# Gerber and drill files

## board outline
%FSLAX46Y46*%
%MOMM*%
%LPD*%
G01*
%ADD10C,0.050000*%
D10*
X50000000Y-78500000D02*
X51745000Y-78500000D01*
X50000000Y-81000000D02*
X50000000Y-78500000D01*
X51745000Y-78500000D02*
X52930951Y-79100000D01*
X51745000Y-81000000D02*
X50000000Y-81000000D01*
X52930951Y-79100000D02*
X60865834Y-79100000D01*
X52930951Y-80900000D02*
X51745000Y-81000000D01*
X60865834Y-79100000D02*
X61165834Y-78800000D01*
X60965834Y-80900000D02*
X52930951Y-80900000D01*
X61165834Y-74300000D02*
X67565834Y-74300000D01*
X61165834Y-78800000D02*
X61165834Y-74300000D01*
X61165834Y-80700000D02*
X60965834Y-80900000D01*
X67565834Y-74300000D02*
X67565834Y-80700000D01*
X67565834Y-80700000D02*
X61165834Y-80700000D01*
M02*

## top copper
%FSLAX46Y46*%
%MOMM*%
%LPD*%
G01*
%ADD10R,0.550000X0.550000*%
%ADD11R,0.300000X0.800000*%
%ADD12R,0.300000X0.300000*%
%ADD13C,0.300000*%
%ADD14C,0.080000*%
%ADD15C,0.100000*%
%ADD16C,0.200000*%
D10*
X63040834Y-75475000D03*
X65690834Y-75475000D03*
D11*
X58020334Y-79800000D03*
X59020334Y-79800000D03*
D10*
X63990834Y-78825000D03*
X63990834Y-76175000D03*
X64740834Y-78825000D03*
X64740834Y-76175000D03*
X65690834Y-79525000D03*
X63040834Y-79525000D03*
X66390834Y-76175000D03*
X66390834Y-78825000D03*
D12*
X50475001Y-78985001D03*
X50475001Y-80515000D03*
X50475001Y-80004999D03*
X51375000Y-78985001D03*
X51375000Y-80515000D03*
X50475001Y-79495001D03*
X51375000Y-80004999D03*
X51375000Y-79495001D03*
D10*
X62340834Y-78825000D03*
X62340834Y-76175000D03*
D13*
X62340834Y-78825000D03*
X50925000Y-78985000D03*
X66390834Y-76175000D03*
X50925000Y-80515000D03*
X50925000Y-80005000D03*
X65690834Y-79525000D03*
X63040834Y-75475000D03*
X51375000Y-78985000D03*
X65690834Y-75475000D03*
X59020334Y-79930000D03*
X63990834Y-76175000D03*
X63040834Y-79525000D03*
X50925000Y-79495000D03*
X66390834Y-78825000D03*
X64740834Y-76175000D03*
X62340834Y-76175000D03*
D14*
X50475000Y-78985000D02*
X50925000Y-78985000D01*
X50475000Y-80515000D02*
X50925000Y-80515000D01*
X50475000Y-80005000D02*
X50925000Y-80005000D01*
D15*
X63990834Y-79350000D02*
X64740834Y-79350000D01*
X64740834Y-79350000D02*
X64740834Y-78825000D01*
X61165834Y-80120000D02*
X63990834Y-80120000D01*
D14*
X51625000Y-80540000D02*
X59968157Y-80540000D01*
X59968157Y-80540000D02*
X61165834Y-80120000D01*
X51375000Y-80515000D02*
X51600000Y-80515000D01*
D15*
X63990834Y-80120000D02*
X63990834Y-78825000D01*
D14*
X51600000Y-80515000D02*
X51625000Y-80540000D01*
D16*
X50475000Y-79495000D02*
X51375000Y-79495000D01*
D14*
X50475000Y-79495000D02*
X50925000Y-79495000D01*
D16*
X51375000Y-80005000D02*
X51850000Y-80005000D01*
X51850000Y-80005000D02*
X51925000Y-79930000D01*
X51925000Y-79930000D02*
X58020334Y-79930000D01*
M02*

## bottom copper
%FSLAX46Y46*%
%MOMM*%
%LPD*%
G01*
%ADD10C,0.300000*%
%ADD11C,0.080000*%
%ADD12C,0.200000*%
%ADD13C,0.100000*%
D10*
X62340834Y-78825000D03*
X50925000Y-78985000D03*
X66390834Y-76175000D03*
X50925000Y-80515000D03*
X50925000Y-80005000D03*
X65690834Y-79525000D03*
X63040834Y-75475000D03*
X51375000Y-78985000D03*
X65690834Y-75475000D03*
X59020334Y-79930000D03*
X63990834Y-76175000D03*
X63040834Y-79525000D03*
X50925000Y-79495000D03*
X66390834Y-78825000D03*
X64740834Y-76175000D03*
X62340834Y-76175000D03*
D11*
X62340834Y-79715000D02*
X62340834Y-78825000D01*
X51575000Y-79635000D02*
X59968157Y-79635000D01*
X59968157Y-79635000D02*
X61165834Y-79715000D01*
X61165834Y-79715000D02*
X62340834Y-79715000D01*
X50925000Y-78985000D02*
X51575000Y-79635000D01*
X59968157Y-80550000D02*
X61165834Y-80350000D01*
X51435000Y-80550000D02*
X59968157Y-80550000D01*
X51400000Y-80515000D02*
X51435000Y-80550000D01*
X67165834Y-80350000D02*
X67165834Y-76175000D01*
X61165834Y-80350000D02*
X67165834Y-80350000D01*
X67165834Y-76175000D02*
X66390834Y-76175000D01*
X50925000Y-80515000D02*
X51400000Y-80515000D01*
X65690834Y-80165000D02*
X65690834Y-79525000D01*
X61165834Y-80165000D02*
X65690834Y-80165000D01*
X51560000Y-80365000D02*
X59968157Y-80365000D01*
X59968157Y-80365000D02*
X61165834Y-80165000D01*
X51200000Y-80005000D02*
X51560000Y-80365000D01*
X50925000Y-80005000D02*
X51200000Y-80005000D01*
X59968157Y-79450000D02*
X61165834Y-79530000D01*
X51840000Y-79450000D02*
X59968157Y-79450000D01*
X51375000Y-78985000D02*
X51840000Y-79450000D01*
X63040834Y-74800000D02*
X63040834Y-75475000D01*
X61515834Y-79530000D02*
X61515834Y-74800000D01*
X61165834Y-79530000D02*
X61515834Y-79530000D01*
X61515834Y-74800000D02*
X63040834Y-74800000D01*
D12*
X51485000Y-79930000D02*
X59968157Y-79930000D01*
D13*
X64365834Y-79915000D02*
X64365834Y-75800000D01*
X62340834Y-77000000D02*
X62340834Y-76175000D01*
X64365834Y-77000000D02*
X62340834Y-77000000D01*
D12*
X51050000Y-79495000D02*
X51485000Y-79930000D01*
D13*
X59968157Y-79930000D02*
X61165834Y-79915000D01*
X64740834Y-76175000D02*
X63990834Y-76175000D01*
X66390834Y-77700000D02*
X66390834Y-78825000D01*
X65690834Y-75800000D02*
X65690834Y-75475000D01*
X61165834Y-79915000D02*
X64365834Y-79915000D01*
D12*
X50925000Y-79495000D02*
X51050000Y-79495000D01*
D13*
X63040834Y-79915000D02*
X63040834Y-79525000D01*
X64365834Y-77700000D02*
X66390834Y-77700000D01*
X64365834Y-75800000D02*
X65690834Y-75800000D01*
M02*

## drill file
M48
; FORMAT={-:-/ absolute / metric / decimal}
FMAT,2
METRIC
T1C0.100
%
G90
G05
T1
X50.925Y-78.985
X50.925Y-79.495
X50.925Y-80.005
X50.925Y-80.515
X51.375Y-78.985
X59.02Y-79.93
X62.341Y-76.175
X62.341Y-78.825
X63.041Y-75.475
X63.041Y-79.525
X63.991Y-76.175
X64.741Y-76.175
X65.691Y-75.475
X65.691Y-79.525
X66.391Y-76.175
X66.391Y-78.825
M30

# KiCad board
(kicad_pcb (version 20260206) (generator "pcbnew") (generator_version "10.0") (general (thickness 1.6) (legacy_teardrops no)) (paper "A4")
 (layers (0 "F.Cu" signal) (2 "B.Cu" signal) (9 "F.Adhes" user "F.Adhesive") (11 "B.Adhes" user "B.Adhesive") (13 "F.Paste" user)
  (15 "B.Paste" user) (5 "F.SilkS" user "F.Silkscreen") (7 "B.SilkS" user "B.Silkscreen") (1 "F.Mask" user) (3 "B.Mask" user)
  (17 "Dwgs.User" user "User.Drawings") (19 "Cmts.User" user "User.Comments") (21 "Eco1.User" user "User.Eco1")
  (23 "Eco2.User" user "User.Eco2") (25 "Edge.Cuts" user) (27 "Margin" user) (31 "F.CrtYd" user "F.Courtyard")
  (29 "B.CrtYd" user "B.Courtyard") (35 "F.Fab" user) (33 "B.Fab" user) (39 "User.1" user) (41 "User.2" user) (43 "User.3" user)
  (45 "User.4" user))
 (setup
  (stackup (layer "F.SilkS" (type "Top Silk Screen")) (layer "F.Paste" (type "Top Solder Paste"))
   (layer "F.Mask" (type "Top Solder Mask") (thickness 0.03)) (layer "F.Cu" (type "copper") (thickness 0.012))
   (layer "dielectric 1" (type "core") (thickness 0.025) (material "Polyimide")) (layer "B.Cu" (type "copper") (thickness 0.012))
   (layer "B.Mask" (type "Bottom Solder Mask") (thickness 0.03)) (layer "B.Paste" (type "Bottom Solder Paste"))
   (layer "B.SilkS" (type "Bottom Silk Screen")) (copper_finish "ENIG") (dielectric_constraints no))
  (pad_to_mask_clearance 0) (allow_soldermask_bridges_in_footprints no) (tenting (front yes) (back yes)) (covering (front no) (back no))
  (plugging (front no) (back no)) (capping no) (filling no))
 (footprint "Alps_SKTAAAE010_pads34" (layer "F.Cu") (at 61.965834 77.5 90)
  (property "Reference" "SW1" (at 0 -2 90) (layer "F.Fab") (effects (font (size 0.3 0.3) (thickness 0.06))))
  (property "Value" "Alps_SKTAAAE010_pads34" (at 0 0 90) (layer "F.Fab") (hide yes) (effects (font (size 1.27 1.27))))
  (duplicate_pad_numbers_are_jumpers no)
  (pad "3" smd rect (at -1.325 0.375 90) (size 0.55 0.55) (layers "F.Cu" "F.Mask") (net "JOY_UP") (solder_mask_margin 0.05)
   (thermal_bridge_angle 45))
  (pad "4" smd rect (at 1.325 0.375 90) (size 0.55 0.55) (layers "F.Cu" "F.Mask") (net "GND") (solder_mask_margin 0.05)
   (thermal_bridge_angle 45)))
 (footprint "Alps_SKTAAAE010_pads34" (layer "F.Cu") (at 66.765834 77.5 -90)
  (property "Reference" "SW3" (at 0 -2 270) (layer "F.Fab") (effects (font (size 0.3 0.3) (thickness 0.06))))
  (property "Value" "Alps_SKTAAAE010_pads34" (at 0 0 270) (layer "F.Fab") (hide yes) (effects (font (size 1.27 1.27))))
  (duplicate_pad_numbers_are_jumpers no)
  (pad "3" smd rect (at -1.325 0.375 270) (size 0.55 0.55) (layers "F.Cu" "F.Mask") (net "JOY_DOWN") (solder_mask_margin 0.05)
   (thermal_bridge_angle 45))
  (pad "4" smd rect (at 1.325 0.375 270) (size 0.55 0.55) (layers "F.Cu" "F.Mask") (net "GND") (solder_mask_margin 0.05)
   (thermal_bridge_angle 45)))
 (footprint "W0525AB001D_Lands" (layer "F.Cu") (at 58.520334 79.93)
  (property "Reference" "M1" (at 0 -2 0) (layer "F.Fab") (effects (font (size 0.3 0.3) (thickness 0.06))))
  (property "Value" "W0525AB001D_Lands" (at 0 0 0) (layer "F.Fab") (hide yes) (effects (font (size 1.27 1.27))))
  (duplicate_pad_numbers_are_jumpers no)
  (pad "1" smd rect (at -0.5 -0.13) (size 0.3 0.8) (layers "F.Cu" "F.Mask") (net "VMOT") (solder_mask_margin 0.05) (thermal_bridge_angle 45))
  (pad "2" smd rect (at 0.5 -0.13) (size 0.3 0.8) (layers "F.Cu" "F.Mask") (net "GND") (solder_mask_margin 0.05) (thermal_bridge_angle 45)))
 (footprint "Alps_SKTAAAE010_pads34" (layer "F.Cu") (at 64.365834 75.1)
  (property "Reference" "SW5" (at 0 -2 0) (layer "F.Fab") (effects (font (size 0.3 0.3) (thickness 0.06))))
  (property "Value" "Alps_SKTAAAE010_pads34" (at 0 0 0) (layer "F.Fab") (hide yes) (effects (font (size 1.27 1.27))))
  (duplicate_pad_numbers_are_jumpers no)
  (pad "3" smd rect (at -1.325 0.375) (size 0.55 0.55) (layers "F.Cu" "F.Mask") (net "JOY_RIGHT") (solder_mask_margin 0.05)
   (thermal_bridge_angle 45))
  (pad "4" smd rect (at 1.325 0.375) (size 0.55 0.55) (layers "F.Cu" "F.Mask") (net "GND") (solder_mask_margin 0.05)
   (thermal_bridge_angle 45)))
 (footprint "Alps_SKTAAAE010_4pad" (layer "F.Cu") (at 64.365834 77.5 90)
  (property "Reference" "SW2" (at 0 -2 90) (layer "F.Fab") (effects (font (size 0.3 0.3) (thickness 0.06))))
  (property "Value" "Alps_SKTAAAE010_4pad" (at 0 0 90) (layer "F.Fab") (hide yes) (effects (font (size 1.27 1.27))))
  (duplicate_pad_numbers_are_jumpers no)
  (pad "1" smd rect (at -1.325 -0.375 90) (size 0.55 0.55) (layers "F.Cu" "F.Mask") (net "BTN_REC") (solder_mask_margin 0.05)
   (thermal_bridge_angle 45))
  (pad "2" smd rect (at 1.325 -0.375 90) (size 0.55 0.55) (layers "F.Cu" "F.Mask") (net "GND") (solder_mask_margin 0.05)
   (thermal_bridge_angle 45))
  (pad "3" smd rect (at -1.325 0.375 90) (size 0.55 0.55) (layers "F.Cu" "F.Mask") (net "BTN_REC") (solder_mask_margin 0.05)
   (thermal_bridge_angle 45))
  (pad "4" smd rect (at 1.325 0.375 90) (size 0.55 0.55) (layers "F.Cu" "F.Mask") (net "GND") (solder_mask_margin 0.05)
   (thermal_bridge_angle 45)))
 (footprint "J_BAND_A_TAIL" (layer "F.Cu") (at 50.9 79.75)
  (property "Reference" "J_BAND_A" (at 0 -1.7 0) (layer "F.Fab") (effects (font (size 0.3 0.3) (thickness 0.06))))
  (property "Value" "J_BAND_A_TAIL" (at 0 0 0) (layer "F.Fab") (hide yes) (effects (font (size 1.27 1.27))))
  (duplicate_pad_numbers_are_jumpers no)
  (pad "1" smd rect (at -0.424999 -0.764999) (size 0.3 0.3) (layers "F.Cu" "F.Mask") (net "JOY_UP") (solder_mask_margin 0.05)
   (thermal_bridge_angle 45))
  (pad "2" smd rect (at -0.424999 0.765) (size 0.3 0.3) (layers "F.Cu" "F.Mask") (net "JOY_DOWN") (solder_mask_margin 0.05)
   (thermal_bridge_angle 45))
  (pad "3" smd rect (at -0.424999 0.254999) (size 0.3 0.3) (layers "F.Cu" "F.Mask") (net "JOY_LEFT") (solder_mask_margin 0.05)
   (thermal_bridge_angle 45))
  (pad "4" smd rect (at 0.475 -0.764999) (size 0.3 0.3) (layers "F.Cu" "F.Mask") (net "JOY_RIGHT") (solder_mask_margin 0.05)
   (thermal_bridge_angle 45))
  (pad "5" smd rect (at 0.475 0.765) (size 0.3 0.3) (layers "F.Cu" "F.Mask") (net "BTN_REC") (solder_mask_margin 0.05)
   (thermal_bridge_angle 45))
  (pad "6" smd rect (at -0.424999 -0.254999) (size 0.3 0.3) (layers "F.Cu" "F.Mask") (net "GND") (solder_mask_margin 0.05)
   (thermal_bridge_angle 45))
  (pad "7" smd rect (at 0.475 0.254999) (size 0.3 0.3) (layers "F.Cu" "F.Mask") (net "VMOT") (solder_mask_margin 0.05)
   (thermal_bridge_angle 45))
  (pad "8" smd rect (at 0.475 -0.254999) (size 0.3 0.3) (layers "F.Cu" "F.Mask") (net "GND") (solder_mask_margin 0.05)
   (thermal_bridge_angle 45)))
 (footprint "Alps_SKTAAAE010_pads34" (layer "F.Cu") (at 64.365834 79.9 180)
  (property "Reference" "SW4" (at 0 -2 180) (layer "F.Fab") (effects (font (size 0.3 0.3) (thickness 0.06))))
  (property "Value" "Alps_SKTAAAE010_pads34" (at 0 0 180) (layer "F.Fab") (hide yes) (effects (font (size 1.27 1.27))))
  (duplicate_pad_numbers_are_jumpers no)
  (pad "3" smd rect (at -1.325 0.375 180) (size 0.55 0.55) (layers "F.Cu" "F.Mask") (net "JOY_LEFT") (solder_mask_margin 0.05)
   (thermal_bridge_angle 45))
  (pad "4" smd rect (at 1.325 0.375 180) (size 0.55 0.55) (layers "F.Cu" "F.Mask") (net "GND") (solder_mask_margin 0.05)
   (thermal_bridge_angle 45)))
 (gr_line (start 50 78.5) (end 51.745 78.5) (stroke (width 0.05) (type default)) (layer "Edge.Cuts"))
 (gr_line (start 50 81) (end 50 78.5) (stroke (width 0.05) (type default)) (layer "Edge.Cuts"))
 (gr_line (start 51.745 78.5) (end 52.930951 79.1) (stroke (width 0.05) (type default)) (layer "Edge.Cuts"))
 (gr_line (start 51.745 81) (end 50 81) (stroke (width 0.05) (type default)) (layer "Edge.Cuts"))
 (gr_line (start 52.930951 79.1) (end 60.865834 79.1) (stroke (width 0.05) (type default)) (layer "Edge.Cuts"))
 (gr_line (start 52.930951 80.9) (end 51.745 81) (stroke (width 0.05) (type default)) (layer "Edge.Cuts"))
 (gr_line (start 60.865834 79.1) (end 61.165834 78.8) (stroke (width 0.05) (type default)) (layer "Edge.Cuts"))
 (gr_line (start 60.965834 80.9) (end 52.930951 80.9) (stroke (width 0.05) (type default)) (layer "Edge.Cuts"))
 (gr_line (start 61.165834 74.3) (end 67.565834 74.3) (stroke (width 0.05) (type default)) (layer "Edge.Cuts"))
 (gr_line (start 61.165834 78.8) (end 61.165834 74.3) (stroke (width 0.05) (type default)) (layer "Edge.Cuts"))
 (gr_line (start 61.165834 80.7) (end 60.965834 80.9) (stroke (width 0.05) (type default)) (layer "Edge.Cuts"))
 (gr_line (start 67.565834 74.3) (end 67.565834 80.7) (stroke (width 0.05) (type default)) (layer "Edge.Cuts"))
 (gr_line (start 67.565834 80.7) (end 61.165834 80.7) (stroke (width 0.05) (type default)) (layer "Edge.Cuts"))
 (segment (start 50.475 78.985) (end 50.925 78.985) (width 0.08) (layer "F.Cu") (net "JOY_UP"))
 (via (at 62.340834 78.825) (size 0.3) (drill 0.1) (layers "F.Cu" "B.Cu") (tenting (front yes) (back yes)) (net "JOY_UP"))
 (via (at 50.925 78.985) (size 0.3) (drill 0.1) (layers "F.Cu" "B.Cu") (tenting (front yes) (back yes)) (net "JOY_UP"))
 (segment (start 61.165834 79.715) (end 62.340834 79.715) (width 0.08) (layer "B.Cu") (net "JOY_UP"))
 (segment (start 50.925 78.985) (end 51.575 79.635) (width 0.08) (layer "B.Cu") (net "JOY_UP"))
 (segment (start 59.968157 79.635) (end 61.165834 79.715) (width 0.08) (layer "B.Cu") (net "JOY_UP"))
 (segment (start 51.575 79.635) (end 59.968157 79.635) (width 0.08) (layer "B.Cu") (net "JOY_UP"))
 (segment (start 62.340834 79.715) (end 62.340834 78.825) (width 0.08) (layer "B.Cu") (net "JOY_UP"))
 (segment (start 50.475 80.515) (end 50.925 80.515) (width 0.08) (layer "F.Cu") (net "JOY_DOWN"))
 (via (at 50.925 80.515) (size 0.3) (drill 0.1) (layers "F.Cu" "B.Cu") (tenting (front yes) (back yes)) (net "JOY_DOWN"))
 (via (at 66.390834 76.175) (size 0.3) (drill 0.1) (layers "F.Cu" "B.Cu") (tenting (front yes) (back yes)) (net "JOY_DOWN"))
 (segment (start 67.165834 80.35) (end 67.165834 76.175) (width 0.08) (layer "B.Cu") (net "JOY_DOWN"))
 (segment (start 51.435 80.55) (end 59.968157 80.55) (width 0.08) (layer "B.Cu") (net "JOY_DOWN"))
 (segment (start 67.165834 76.175) (end 66.390834 76.175) (width 0.08) (layer "B.Cu") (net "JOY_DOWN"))
 (segment (start 61.165834 80.35) (end 67.165834 80.35) (width 0.08) (layer "B.Cu") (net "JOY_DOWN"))
 (segment (start 59.968157 80.55) (end 61.165834 80.35) (width 0.08) (layer "B.Cu") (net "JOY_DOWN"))
 (segment (start 51.4 80.515) (end 51.435 80.55) (width 0.08) (layer "B.Cu") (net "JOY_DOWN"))
 (segment (start 50.925 80.515) (end 51.4 80.515) (width 0.08) (layer "B.Cu") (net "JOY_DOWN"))
 (segment (start 50.475 80.005) (end 50.925 80.005) (width 0.08) (layer "F.Cu") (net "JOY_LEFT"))
 (via (at 50.925 80.005) (size 0.3) (drill 0.1) (layers "F.Cu" "B.Cu") (tenting (front yes) (back yes)) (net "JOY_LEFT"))
 (via (at 65.690834 79.525) (size 0.3) (drill 0.1) (layers "F.Cu" "B.Cu") (tenting (front yes) (back yes)) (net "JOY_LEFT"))
 (segment (start 65.690834 80.165) (end 65.690834 79.525) (width 0.08) (layer "B.Cu") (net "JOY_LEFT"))
 (segment (start 61.165834 80.165) (end 65.690834 80.165) (width 0.08) (layer "B.Cu") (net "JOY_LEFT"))
 (segment (start 51.56 80.365) (end 59.968157 80.365) (width 0.08) (layer "B.Cu") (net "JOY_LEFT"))
 (segment (start 51.2 80.005) (end 51.56 80.365) (width 0.08) (layer "B.Cu") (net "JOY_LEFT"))
 (segment (start 50.925 80.005) (end 51.2 80.005) (width 0.08) (layer "B.Cu") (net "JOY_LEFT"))
 (segment (start 59.968157 80.365) (end 61.165834 80.165) (width 0.08) (layer "B.Cu") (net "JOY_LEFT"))
 (via (at 63.040834 75.475) (size 0.3) (drill 0.1) (layers "F.Cu" "B.Cu") (tenting (front yes) (back yes)) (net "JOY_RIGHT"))
 (via (at 51.375 78.985) (size 0.3) (drill 0.1) (layers "F.Cu" "B.Cu") (tenting (front yes) (back yes)) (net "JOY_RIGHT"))
 (segment (start 51.375 78.985) (end 51.84 79.45) (width 0.08) (layer "B.Cu") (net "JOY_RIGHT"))
 (segment (start 51.84 79.45) (end 59.968157 79.45) (width 0.08) (layer "B.Cu") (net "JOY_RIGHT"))
 (segment (start 63.040834 74.8) (end 63.040834 75.475) (width 0.08) (layer "B.Cu") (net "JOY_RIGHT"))
 (segment (start 61.515834 74.8) (end 63.040834 74.8) (width 0.08) (layer "B.Cu") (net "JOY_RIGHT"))
 (segment (start 59.968157 79.45) (end 61.165834 79.53) (width 0.08) (layer "B.Cu") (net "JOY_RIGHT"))
 (segment (start 61.165834 79.53) (end 61.515834 79.53) (width 0.08) (layer "B.Cu") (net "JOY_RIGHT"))
 (segment (start 61.515834 79.53) (end 61.515834 74.8) (width 0.08) (layer "B.Cu") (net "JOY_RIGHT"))
 (segment (start 51.6 80.515) (end 51.625 80.54) (width 0.08) (layer "F.Cu") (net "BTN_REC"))
 (segment (start 51.375 80.515) (end 51.6 80.515) (width 0.08) (layer "F.Cu") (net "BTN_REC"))
 (segment (start 64.740834 79.35) (end 64.740834 78.825) (width 0.1) (layer "F.Cu") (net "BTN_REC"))
 (segment (start 61.165834 80.12) (end 63.990834 80.12) (width 0.1) (layer "F.Cu") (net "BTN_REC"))
 (segment (start 51.625 80.54) (end 59.968157 80.54) (width 0.08) (layer "F.Cu") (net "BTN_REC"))
 (segment (start 63.990834 80.12) (end 63.990834 78.825) (width 0.1) (layer "F.Cu") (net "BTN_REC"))
 (segment (start 59.968157 80.54) (end 61.165834 80.12) (width 0.08) (layer "F.Cu") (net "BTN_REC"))
 (segment (start 63.990834 79.35) (end 64.740834 79.35) (width 0.1) (layer "F.Cu") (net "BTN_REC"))
 (segment (start 50.475 79.495) (end 51.375 79.495) (width 0.2) (layer "F.Cu") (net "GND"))
 (segment (start 50.475 79.495) (end 50.925 79.495) (width 0.08) (layer "F.Cu") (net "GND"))
 (via (at 62.340834 76.175) (size 0.3) (drill 0.1) (layers "F.Cu" "B.Cu") (tenting (front yes) (back yes)) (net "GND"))
 (via (at 64.740834 76.175) (size 0.3) (drill 0.1) (layers "F.Cu" "B.Cu") (tenting (front yes) (back yes)) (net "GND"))
 (via (at 59.020334 79.93) (size 0.3) (drill 0.1) (layers "F.Cu" "B.Cu") (tenting (front yes) (back yes)) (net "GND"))
 (via (at 50.925 79.495) (size 0.3) (drill 0.1) (layers "F.Cu" "B.Cu") (tenting (front yes) (back yes)) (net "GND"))
 (via (at 63.040834 79.525) (size 0.3) (drill 0.1) (layers "F.Cu" "B.Cu") (tenting (front yes) (back yes)) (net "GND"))
 (via (at 63.990834 76.175) (size 0.3) (drill 0.1) (layers "F.Cu" "B.Cu") (tenting (front yes) (back yes)) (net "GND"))
 (via (at 66.390834 78.825) (size 0.3) (drill 0.1) (layers "F.Cu" "B.Cu") (tenting (front yes) (back yes)) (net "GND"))
 (via (at 65.690834 75.475) (size 0.3) (drill 0.1) (layers "F.Cu" "B.Cu") (tenting (front yes) (back yes)) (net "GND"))
 (segment (start 59.968157 79.93) (end 61.165834 79.915) (width 0.1) (layer "B.Cu") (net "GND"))
 (segment (start 63.040834 79.915) (end 63.040834 79.525) (width 0.1) (layer "B.Cu") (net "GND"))
 (segment (start 62.340834 77) (end 62.340834 76.175) (width 0.1) (layer "B.Cu") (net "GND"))
 (segment (start 64.365834 77) (end 62.340834 77) (width 0.1) (layer "B.Cu") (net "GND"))
 (segment (start 66.390834 77.7) (end 66.390834 78.825) (width 0.1) (layer "B.Cu") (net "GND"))
 (segment (start 51.485 79.93) (end 59.968157 79.93) (width 0.2) (layer "B.Cu") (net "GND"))
 (segment (start 65.690834 75.8) (end 65.690834 75.475) (width 0.1) (layer "B.Cu") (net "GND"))
 (segment (start 50.925 79.495) (end 51.05 79.495) (width 0.2) (layer "B.Cu") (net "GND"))
 (segment (start 64.365834 75.8) (end 65.690834 75.8) (width 0.1) (layer "B.Cu") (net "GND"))
 (segment (start 64.365834 77.7) (end 66.390834 77.7) (width 0.1) (layer "B.Cu") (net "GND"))
 (segment (start 64.740834 76.175) (end 63.990834 76.175) (width 0.1) (layer "B.Cu") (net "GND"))
 (segment (start 64.365834 79.915) (end 64.365834 75.8) (width 0.1) (layer "B.Cu") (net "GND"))
 (segment (start 61.165834 79.915) (end 64.365834 79.915) (width 0.1) (layer "B.Cu") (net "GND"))
 (segment (start 51.05 79.495) (end 51.485 79.93) (width 0.2) (layer "B.Cu") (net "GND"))
 (segment (start 51.925 79.93) (end 58.020334 79.93) (width 0.2) (layer "F.Cu") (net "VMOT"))
 (segment (start 51.375 80.005) (end 51.85 80.005) (width 0.2) (layer "F.Cu") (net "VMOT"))
 (segment (start 51.85 80.005) (end 51.925 79.93) (width 0.2) (layer "F.Cu") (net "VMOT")))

